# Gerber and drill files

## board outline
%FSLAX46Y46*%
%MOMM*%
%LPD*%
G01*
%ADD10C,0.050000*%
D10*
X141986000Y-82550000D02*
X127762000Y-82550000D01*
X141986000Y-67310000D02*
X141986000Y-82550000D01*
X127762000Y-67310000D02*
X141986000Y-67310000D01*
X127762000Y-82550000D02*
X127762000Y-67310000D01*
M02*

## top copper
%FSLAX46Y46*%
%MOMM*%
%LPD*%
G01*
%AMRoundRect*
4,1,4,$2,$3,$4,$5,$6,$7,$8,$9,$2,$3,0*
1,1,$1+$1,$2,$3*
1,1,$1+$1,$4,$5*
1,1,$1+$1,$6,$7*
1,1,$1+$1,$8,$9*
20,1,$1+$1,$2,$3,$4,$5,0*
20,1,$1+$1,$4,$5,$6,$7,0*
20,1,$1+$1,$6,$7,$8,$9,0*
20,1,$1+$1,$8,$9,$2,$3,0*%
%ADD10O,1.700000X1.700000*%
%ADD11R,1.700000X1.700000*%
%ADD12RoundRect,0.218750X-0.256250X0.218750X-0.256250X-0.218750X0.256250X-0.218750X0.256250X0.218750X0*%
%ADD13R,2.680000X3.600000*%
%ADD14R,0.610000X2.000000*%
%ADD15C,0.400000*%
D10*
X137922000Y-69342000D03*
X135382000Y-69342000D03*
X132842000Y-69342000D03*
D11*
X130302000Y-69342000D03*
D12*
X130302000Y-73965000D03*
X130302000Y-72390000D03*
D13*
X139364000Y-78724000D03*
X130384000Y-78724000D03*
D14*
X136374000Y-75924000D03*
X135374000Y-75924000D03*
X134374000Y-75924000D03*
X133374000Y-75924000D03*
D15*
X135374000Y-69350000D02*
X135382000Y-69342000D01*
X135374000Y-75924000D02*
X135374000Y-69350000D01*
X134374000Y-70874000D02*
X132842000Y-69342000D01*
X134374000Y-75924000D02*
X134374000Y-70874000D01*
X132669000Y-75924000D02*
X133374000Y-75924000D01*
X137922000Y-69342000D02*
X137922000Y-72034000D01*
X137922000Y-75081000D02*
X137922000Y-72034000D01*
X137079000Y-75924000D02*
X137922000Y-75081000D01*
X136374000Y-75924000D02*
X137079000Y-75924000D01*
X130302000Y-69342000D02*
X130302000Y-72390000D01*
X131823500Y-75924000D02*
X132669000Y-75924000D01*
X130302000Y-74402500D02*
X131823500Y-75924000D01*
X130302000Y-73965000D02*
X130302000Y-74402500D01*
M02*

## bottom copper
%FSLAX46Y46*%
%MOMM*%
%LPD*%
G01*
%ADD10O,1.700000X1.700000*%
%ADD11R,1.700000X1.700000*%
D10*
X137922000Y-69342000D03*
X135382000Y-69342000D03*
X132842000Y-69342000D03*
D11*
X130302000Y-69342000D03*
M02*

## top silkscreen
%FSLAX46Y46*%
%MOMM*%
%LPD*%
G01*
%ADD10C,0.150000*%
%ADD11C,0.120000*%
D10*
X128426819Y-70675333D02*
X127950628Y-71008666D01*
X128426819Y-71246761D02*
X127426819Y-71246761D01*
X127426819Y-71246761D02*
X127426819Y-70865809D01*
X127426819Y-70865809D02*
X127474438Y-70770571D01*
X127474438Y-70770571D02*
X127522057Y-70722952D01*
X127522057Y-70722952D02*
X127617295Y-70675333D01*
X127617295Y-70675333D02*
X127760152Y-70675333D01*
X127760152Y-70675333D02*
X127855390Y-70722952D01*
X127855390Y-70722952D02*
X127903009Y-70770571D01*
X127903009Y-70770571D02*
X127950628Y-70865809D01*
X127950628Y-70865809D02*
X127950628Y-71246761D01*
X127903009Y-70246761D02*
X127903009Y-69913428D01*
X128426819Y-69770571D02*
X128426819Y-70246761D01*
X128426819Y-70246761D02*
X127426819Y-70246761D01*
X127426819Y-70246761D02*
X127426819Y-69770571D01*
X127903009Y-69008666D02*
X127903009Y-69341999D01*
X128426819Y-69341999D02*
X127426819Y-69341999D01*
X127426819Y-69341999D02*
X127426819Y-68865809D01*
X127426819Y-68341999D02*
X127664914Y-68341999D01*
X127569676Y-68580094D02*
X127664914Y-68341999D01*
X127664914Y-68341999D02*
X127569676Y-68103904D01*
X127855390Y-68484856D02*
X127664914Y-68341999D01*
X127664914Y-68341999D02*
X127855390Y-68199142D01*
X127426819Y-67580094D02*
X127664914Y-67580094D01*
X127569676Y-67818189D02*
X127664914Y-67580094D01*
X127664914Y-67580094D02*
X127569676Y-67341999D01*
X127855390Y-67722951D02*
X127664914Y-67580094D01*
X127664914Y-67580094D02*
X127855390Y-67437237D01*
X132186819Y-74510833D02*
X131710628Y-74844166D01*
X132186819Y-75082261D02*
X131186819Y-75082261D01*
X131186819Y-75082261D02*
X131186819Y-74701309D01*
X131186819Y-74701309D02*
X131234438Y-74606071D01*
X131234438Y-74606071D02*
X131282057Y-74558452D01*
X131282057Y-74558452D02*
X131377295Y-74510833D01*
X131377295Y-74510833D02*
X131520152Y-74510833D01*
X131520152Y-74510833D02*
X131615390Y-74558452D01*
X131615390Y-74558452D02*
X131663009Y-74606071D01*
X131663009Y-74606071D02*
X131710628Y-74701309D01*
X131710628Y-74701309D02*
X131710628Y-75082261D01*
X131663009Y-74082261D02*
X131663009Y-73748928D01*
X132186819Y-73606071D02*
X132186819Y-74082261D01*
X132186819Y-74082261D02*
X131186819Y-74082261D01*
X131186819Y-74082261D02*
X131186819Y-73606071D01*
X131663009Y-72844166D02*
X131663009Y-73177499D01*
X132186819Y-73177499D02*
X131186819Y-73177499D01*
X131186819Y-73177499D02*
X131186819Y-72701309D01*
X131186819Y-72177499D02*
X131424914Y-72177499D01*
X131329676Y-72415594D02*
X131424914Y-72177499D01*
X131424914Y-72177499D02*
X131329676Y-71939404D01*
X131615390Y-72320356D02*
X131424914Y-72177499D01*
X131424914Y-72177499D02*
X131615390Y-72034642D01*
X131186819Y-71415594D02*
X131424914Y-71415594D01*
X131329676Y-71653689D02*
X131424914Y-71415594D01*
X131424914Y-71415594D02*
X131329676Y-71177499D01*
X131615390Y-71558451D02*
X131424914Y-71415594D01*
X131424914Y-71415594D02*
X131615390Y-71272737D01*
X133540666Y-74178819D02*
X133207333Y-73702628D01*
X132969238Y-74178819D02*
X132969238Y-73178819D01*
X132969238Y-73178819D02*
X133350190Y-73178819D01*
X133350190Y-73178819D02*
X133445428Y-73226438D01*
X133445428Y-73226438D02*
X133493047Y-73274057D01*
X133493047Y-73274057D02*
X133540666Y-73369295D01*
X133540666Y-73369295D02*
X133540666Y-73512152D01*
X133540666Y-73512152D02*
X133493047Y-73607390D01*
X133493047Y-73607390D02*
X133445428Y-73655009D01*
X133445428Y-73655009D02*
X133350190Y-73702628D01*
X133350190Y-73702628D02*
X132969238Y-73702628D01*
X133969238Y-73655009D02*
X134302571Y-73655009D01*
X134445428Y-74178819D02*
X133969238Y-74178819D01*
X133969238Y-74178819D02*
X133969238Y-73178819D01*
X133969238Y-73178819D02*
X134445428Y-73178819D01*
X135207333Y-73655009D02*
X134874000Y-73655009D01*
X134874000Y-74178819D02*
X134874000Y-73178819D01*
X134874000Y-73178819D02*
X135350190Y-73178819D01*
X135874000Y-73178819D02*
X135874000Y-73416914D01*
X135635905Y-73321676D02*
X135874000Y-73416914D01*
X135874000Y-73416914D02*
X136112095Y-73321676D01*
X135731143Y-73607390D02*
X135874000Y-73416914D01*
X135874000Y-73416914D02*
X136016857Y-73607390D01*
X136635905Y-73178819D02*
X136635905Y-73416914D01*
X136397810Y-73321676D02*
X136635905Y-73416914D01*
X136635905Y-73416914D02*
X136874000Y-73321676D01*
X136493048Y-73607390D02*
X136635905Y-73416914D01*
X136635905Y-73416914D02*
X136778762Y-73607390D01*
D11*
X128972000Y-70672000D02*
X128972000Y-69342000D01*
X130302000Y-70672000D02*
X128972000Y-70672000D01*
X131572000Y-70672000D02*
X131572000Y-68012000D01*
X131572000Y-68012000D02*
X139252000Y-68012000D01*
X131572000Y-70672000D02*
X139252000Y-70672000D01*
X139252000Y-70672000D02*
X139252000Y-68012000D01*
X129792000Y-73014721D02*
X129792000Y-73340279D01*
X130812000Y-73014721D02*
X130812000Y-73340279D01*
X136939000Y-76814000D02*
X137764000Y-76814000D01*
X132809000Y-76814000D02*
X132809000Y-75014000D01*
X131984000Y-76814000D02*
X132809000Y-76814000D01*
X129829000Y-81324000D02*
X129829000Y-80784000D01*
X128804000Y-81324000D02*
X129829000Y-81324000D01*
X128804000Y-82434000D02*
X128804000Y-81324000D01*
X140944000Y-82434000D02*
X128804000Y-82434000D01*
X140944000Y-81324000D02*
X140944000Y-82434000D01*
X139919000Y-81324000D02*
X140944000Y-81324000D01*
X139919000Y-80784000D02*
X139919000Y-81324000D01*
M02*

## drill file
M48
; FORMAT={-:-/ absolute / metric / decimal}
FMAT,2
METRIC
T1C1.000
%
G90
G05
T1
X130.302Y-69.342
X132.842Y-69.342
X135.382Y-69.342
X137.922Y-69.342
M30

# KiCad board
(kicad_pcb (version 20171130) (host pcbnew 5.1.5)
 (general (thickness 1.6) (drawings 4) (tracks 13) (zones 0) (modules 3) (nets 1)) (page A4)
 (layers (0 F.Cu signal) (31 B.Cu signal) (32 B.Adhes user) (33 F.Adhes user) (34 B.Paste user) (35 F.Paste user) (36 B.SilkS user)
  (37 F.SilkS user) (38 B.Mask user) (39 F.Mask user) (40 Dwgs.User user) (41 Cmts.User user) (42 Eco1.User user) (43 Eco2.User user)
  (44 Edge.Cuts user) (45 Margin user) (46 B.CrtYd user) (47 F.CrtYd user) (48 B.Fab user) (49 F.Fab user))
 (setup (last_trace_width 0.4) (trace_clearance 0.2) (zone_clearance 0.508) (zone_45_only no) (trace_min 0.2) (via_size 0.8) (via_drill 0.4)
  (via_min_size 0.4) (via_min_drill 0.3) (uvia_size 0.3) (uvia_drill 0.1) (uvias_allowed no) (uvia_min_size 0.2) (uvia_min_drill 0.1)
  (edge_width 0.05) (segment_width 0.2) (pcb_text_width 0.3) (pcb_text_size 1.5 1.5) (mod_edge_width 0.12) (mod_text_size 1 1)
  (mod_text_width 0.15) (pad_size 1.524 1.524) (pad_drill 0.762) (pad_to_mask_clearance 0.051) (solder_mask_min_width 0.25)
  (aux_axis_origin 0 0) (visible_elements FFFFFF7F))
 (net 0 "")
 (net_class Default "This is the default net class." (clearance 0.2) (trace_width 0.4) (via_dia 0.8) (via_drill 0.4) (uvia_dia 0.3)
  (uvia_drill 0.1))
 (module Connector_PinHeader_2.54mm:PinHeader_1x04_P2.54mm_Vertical (layer F.Cu) (at 130.302 69.342 90)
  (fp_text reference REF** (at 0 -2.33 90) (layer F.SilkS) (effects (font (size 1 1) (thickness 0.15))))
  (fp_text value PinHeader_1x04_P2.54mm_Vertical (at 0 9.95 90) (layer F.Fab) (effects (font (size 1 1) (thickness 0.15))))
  (fp_line (start -1.33 -1.33) (end 0 -1.33) (layer F.SilkS) (width 0.12))
  (fp_line (start -1.33 0) (end -1.33 -1.33) (layer F.SilkS) (width 0.12))
  (fp_line (start -1.33 1.27) (end 1.33 1.27) (layer F.SilkS) (width 0.12))
  (fp_line (start 1.33 1.27) (end 1.33 8.95) (layer F.SilkS) (width 0.12))
  (fp_line (start -1.33 1.27) (end -1.33 8.95) (layer F.SilkS) (width 0.12))
  (fp_line (start -1.33 8.95) (end 1.33 8.95) (layer F.SilkS) (width 0.12))
  (pad 4 thru_hole oval (at 0 7.62 90) (size 1.7 1.7) (drill 1) (layers *.Cu *.Mask))
  (pad 3 thru_hole oval (at 0 5.08 90) (size 1.7 1.7) (drill 1) (layers *.Cu *.Mask))
  (pad 2 thru_hole oval (at 0 2.54 90) (size 1.7 1.7) (drill 1) (layers *.Cu *.Mask))
  (pad 1 thru_hole rect (at 0 0 90) (size 1.7 1.7) (drill 1) (layers *.Cu *.Mask)))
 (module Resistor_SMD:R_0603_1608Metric (layer F.Cu) (at 130.302 73.1775 270)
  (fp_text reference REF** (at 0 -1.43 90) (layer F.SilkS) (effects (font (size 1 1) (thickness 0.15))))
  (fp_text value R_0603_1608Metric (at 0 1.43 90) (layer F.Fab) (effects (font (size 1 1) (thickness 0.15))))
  (fp_line (start -0.162779 0.51) (end 0.162779 0.51) (layer F.SilkS) (width 0.12))
  (fp_line (start -0.162779 -0.51) (end 0.162779 -0.51) (layer F.SilkS) (width 0.12))
  (pad 2 smd roundrect (at 0.7875 0 270) (size 0.875 0.95) (layers F.Cu F.Paste F.Mask) (roundrect_rratio 0.25))
  (pad 1 smd roundrect (at -0.7875 0 270) (size 0.875 0.95) (layers F.Cu F.Paste F.Mask) (roundrect_rratio 0.25)))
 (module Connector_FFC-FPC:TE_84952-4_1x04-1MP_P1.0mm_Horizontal (layer F.Cu) (at 134.874 77.724)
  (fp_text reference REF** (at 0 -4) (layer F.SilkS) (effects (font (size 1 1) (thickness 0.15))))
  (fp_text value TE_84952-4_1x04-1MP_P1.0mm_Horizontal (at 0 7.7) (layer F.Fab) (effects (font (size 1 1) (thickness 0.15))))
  (fp_line (start 2.065 -0.91) (end 2.89 -0.91) (layer F.SilkS) (width 0.12))
  (fp_line (start -2.065 -0.91) (end -2.065 -2.71) (layer F.SilkS) (width 0.12))
  (fp_line (start -2.89 -0.91) (end -2.065 -0.91) (layer F.SilkS) (width 0.12))
  (fp_line (start -5.045 3.6) (end -5.045 3.06) (layer F.SilkS) (width 0.12))
  (fp_line (start -6.07 3.6) (end -5.045 3.6) (layer F.SilkS) (width 0.12))
  (fp_line (start -6.07 4.71) (end -6.07 3.6) (layer F.SilkS) (width 0.12))
  (fp_line (start 6.07 4.71) (end -6.07 4.71) (layer F.SilkS) (width 0.12))
  (fp_line (start 6.07 3.6) (end 6.07 4.71) (layer F.SilkS) (width 0.12))
  (fp_line (start 5.045 3.6) (end 6.07 3.6) (layer F.SilkS) (width 0.12))
  (fp_line (start 5.045 3.06) (end 5.045 3.6) (layer F.SilkS) (width 0.12))
  (pad MP smd rect (at 4.49 1) (size 2.68 3.6) (layers F.Cu F.Paste F.Mask))
  (pad MP smd rect (at -4.49 1) (size 2.68 3.6) (layers F.Cu F.Paste F.Mask))
  (pad 4 smd rect (at 1.5 -1.8) (size 0.61 2) (layers F.Cu F.Paste F.Mask))
  (pad 3 smd rect (at 0.5 -1.8) (size 0.61 2) (layers F.Cu F.Paste F.Mask))
  (pad 2 smd rect (at -0.5 -1.8) (size 0.61 2) (layers F.Cu F.Paste F.Mask))
  (pad 1 smd rect (at -1.5 -1.8) (size 0.61 2) (layers F.Cu F.Paste F.Mask)))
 (gr_line (start 141.986 82.55) (end 127.762 82.55) (layer Edge.Cuts) (width 0.05))
 (gr_line (start 141.986 67.31) (end 141.986 82.55) (layer Edge.Cuts) (width 0.05))
 (gr_line (start 127.762 67.31) (end 141.986 67.31) (layer Edge.Cuts) (width 0.05))
 (gr_line (start 127.762 82.55) (end 127.762 67.31) (layer Edge.Cuts) (width 0.05))
 (segment (start 135.374 69.35) (end 135.382 69.342) (width 0.4) (layer F.Cu) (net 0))
 (segment (start 135.374 75.924) (end 135.374 69.35) (width 0.4) (layer F.Cu) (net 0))
 (segment (start 134.374 70.874) (end 132.842 69.342) (width 0.4) (layer F.Cu) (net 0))
 (segment (start 134.374 75.924) (end 134.374 70.874) (width 0.4) (layer F.Cu) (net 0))
 (segment (start 132.669 75.924) (end 133.374 75.924) (width 0.4) (layer F.Cu) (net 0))
 (segment (start 137.922 69.342) (end 137.922 72.034) (width 0.4) (layer F.Cu) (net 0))
 (segment (start 137.922 75.081) (end 137.922 72.034) (width 0.4) (layer F.Cu) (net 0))
 (segment (start 137.079 75.924) (end 137.922 75.081) (width 0.4) (layer F.Cu) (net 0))
 (segment (start 136.374 75.924) (end 137.079 75.924) (width 0.4) (layer F.Cu) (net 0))
 (segment (start 130.302 69.342) (end 130.302 72.39) (width 0.4) (layer F.Cu) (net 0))
 (segment (start 131.8235 75.924) (end 132.669 75.924) (width 0.4) (layer F.Cu) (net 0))
 (segment (start 130.302 74.4025) (end 131.8235 75.924) (width 0.4) (layer F.Cu) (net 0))
 (segment (start 130.302 73.965) (end 130.302 74.4025) (width 0.4) (layer F.Cu) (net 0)))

